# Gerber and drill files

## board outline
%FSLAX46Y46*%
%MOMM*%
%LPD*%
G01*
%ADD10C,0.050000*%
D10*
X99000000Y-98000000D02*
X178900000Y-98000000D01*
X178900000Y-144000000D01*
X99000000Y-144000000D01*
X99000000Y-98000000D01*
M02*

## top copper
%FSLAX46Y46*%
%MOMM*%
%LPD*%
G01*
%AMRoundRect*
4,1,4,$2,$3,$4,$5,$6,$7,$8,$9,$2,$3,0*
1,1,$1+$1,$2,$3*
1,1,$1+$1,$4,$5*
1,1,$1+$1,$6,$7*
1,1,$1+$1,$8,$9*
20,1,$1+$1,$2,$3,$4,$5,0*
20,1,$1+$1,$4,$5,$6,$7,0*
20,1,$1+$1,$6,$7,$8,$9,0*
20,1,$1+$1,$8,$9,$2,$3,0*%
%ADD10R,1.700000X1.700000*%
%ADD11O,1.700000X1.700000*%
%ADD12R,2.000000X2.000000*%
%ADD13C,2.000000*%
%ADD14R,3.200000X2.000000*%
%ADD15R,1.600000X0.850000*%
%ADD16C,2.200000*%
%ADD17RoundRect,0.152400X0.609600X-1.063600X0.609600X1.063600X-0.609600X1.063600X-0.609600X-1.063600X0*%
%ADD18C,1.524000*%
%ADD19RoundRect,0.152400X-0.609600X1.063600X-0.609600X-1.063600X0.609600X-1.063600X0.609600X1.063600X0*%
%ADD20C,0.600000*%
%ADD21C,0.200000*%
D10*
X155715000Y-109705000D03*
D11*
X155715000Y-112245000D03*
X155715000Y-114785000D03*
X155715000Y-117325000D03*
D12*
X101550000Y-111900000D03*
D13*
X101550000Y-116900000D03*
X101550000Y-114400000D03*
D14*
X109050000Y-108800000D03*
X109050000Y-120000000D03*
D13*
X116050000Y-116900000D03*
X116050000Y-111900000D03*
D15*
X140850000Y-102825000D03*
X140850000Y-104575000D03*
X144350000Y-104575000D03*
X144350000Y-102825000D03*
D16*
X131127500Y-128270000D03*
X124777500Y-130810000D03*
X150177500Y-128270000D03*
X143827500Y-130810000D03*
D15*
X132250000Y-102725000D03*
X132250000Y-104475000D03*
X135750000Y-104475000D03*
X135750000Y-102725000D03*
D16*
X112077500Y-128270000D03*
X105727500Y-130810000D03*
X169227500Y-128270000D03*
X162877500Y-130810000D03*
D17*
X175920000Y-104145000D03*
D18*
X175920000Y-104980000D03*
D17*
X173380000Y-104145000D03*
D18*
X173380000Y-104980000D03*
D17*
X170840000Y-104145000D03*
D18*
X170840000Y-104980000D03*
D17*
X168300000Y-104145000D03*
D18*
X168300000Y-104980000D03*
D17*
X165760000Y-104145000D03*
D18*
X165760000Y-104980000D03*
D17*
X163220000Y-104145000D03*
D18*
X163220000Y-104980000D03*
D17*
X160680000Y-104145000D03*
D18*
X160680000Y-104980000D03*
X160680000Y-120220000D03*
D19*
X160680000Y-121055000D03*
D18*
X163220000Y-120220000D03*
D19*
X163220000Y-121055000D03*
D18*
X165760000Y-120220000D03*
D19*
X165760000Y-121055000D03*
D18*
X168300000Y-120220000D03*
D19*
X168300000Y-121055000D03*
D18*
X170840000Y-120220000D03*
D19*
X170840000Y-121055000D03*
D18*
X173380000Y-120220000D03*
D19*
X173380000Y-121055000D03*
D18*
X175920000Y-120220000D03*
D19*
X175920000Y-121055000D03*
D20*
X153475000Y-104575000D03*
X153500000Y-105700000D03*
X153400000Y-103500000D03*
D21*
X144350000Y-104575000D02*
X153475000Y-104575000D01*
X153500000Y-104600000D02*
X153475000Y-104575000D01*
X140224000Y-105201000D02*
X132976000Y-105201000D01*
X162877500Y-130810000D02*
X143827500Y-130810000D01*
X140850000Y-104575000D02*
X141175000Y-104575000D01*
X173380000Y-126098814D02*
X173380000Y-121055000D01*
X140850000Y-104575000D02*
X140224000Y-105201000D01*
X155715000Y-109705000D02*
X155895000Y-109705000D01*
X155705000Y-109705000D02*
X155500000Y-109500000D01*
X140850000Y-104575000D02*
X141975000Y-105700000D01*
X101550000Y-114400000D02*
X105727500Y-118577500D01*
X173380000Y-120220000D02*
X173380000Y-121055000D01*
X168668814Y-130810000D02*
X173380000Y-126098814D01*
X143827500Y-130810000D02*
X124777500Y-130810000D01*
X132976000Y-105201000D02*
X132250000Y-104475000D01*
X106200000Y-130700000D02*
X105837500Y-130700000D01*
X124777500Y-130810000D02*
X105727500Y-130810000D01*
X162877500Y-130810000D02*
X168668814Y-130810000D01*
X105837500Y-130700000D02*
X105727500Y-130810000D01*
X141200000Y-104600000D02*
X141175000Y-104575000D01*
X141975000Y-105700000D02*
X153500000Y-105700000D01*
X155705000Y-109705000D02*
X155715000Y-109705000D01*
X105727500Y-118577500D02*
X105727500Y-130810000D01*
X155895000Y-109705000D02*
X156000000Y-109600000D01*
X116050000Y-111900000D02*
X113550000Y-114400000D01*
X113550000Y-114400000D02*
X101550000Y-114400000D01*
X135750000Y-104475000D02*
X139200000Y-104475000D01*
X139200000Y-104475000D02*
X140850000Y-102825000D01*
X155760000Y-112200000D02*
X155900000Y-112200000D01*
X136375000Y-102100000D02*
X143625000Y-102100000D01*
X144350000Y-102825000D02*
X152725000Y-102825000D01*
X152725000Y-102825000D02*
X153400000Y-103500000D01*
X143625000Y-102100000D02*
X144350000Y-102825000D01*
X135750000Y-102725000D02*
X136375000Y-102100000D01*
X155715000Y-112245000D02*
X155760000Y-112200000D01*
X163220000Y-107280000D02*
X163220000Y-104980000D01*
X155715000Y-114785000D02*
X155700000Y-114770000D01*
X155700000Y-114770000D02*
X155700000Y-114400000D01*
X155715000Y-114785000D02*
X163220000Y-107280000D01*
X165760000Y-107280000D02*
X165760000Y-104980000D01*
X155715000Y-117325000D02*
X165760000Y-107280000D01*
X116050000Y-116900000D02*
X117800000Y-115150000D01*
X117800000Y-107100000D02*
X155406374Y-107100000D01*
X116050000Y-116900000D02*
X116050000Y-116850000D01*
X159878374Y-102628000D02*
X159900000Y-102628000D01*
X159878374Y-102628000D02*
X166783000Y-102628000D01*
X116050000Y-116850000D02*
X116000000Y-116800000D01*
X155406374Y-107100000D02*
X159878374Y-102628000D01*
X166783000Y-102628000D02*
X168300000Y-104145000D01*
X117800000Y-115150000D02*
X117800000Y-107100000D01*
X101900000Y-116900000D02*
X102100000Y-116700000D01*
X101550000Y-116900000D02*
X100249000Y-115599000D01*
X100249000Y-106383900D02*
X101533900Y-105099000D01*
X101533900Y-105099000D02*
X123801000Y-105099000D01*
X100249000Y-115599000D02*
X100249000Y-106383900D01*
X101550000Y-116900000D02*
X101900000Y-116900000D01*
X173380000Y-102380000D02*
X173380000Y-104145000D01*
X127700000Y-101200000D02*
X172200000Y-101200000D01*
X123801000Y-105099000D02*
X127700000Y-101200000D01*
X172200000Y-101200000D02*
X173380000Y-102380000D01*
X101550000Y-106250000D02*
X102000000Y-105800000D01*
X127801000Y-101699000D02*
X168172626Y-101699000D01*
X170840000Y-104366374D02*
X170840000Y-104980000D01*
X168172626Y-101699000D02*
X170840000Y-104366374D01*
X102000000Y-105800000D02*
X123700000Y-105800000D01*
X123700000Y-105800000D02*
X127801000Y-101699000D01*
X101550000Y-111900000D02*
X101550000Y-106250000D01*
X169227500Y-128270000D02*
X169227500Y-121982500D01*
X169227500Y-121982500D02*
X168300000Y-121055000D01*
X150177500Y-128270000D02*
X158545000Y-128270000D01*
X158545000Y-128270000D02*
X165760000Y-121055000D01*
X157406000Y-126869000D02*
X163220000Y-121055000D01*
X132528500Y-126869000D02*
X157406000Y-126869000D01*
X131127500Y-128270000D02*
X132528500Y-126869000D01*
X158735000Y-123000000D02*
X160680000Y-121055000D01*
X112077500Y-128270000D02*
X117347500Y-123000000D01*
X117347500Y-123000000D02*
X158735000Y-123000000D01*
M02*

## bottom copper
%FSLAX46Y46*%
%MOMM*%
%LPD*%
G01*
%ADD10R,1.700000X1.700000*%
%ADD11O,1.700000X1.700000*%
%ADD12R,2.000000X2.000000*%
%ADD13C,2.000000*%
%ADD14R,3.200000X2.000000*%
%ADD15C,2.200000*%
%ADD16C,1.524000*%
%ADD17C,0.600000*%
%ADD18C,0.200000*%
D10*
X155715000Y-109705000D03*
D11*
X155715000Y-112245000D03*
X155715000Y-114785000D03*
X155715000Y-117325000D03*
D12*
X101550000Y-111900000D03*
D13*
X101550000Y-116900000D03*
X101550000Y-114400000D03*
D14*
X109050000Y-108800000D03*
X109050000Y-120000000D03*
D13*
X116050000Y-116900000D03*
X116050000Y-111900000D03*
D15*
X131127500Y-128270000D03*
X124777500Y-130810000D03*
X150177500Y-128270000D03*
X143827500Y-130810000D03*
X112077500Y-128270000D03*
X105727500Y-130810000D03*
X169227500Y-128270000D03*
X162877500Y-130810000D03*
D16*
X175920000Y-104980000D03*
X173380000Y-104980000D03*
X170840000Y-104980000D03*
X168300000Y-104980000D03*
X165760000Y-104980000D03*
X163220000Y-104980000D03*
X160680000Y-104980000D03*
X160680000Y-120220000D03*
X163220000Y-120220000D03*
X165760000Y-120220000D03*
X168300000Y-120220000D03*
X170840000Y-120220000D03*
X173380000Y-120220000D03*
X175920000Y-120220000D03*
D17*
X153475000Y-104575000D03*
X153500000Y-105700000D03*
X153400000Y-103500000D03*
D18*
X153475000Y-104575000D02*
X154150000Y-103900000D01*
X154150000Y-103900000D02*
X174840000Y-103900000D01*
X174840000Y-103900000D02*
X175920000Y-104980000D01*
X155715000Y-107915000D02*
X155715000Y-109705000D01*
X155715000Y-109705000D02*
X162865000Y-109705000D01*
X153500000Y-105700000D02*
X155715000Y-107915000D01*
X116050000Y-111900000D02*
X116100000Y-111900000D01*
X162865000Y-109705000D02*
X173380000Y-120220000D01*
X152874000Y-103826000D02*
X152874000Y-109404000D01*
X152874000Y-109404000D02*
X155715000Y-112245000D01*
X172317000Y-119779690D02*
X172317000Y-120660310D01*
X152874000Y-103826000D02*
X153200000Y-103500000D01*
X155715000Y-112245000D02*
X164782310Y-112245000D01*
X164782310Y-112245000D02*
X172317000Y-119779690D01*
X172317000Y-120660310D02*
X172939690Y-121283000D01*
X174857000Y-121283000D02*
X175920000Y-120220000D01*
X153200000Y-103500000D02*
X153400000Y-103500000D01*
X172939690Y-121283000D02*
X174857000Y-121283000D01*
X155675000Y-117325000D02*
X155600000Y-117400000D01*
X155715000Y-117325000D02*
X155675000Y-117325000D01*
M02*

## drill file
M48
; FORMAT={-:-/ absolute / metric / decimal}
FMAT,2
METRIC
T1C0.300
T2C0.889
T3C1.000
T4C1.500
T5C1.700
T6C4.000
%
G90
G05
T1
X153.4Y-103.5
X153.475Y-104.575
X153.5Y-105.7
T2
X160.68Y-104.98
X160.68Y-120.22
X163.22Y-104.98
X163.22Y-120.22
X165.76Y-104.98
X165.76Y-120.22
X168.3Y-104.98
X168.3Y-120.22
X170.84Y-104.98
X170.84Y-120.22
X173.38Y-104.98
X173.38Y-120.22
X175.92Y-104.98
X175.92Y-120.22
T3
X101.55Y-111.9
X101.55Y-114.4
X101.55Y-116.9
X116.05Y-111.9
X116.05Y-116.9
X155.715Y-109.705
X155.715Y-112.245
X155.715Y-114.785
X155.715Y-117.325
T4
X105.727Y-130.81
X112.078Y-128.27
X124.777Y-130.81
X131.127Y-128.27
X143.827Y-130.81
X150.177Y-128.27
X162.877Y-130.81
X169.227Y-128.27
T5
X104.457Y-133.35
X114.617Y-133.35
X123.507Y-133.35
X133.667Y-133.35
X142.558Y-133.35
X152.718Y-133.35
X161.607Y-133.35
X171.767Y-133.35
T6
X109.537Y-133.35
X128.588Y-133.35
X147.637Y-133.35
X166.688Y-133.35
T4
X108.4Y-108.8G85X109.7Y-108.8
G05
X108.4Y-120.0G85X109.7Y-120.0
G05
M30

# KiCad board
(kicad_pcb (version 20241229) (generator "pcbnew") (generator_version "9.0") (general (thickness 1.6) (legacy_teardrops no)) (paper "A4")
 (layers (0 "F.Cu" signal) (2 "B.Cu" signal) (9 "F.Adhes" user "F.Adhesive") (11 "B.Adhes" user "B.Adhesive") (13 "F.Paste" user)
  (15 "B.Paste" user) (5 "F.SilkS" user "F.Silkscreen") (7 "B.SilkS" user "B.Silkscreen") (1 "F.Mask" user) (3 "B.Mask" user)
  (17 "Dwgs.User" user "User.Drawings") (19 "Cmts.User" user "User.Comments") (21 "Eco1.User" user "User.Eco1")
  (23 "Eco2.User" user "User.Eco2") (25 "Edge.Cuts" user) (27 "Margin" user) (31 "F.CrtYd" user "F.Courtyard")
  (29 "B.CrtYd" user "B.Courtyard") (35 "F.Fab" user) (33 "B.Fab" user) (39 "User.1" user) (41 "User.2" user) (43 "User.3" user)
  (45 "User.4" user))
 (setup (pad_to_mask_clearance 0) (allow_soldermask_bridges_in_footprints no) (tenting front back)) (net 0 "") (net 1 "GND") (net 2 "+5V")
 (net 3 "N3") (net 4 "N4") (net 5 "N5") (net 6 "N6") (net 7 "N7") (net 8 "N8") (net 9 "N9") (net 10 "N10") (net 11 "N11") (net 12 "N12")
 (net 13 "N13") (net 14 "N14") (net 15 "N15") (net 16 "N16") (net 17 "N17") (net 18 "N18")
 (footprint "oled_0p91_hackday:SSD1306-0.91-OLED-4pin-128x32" (layer "F.Cu") (at 119.215 107.515)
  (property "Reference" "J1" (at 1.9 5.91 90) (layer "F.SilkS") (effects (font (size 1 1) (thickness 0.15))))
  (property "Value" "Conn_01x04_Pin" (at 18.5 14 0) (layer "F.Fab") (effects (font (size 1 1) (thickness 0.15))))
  (pad "1" thru_hole rect (at 36.5 2.19) (size 1.7 1.7) (drill 1) (layers "*.Cu" "*.Mask") (remove_unused_layers no) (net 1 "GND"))
  (pad "2" thru_hole oval (at 36.5 4.73) (size 1.7 1.7) (drill 1) (layers "*.Cu" "*.Mask") (remove_unused_layers no) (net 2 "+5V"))
  (pad "3" thru_hole oval (at 36.5 7.27) (size 1.7 1.7) (drill 1) (layers "*.Cu" "*.Mask") (remove_unused_layers no) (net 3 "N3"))
  (pad "4" thru_hole oval (at 36.5 9.81) (size 1.7 1.7) (drill 1) (layers "*.Cu" "*.Mask") (remove_unused_layers no) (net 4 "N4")))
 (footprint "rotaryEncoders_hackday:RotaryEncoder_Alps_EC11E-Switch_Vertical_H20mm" (layer "F.Cu") (at 101.55 111.9)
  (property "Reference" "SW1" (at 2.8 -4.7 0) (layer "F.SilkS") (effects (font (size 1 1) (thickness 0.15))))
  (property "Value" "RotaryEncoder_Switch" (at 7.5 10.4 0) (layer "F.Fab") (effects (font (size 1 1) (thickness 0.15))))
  (pad "A" thru_hole rect (at 0 0) (size 2 2) (drill 1) (layers "*.Cu" "*.Mask") (remove_unused_layers no) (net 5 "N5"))
  (pad "B" thru_hole circle (at 0 5) (size 2 2) (drill 1) (layers "*.Cu" "*.Mask") (remove_unused_layers no) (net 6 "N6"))
  (pad "C" thru_hole circle (at 0 2.5) (size 2 2) (drill 1) (layers "*.Cu" "*.Mask") (remove_unused_layers no) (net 1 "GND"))
  (pad "MP" thru_hole rect (at 7.5 -3.1) (size 3.2 2) (drill oval 2.8 1.5) (layers "*.Cu" "*.Mask") (remove_unused_layers no))
  (pad "MP" thru_hole rect (at 7.5 8.1) (size 3.2 2) (drill oval 2.8 1.5) (layers "*.Cu" "*.Mask") (remove_unused_layers no))
  (pad "S1" thru_hole circle (at 14.5 5) (size 2 2) (drill 1) (layers "*.Cu" "*.Mask") (remove_unused_layers no) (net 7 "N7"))
  (pad "S2" thru_hole circle (at 14.5 0) (size 2 2) (drill 1) (layers "*.Cu" "*.Mask") (remove_unused_layers no) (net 1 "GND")))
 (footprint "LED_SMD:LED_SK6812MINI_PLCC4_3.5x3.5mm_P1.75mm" (layer "F.Cu") (at 142.6 103.7)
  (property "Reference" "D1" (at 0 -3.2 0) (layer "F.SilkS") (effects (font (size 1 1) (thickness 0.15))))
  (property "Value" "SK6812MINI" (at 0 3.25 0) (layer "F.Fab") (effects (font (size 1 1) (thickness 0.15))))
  (pad "1" smd rect (at -1.75 -0.875) (size 1.6 0.85) (layers "F.Cu" "F.Mask" "F.Paste") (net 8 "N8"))
  (pad "2" smd rect (at -1.75 0.875) (size 1.6 0.85) (layers "F.Cu" "F.Mask" "F.Paste") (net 1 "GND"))
  (pad "3" smd rect (at 1.75 0.875) (size 1.6 0.85) (layers "F.Cu" "F.Mask" "F.Paste") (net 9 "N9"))
  (pad "4" smd rect (at 1.75 -0.875) (size 1.6 0.85) (layers "F.Cu" "F.Mask" "F.Paste") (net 2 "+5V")))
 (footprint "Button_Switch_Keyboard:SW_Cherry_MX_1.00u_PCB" (layer "F.Cu") (at 131.1275 128.27)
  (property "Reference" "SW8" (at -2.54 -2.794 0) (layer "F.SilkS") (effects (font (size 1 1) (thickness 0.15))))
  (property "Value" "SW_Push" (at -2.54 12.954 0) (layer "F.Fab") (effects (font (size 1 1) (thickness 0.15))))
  (pad "" np_thru_hole circle (at -7.62 5.08) (size 1.7 1.7) (drill 1.7) (layers "*.Cu" "*.Mask"))
  (pad "" np_thru_hole circle (at -2.54 5.08) (size 4 4) (drill 4) (layers "*.Cu" "*.Mask"))
  (pad "" np_thru_hole circle (at 2.54 5.08) (size 1.7 1.7) (drill 1.7) (layers "*.Cu" "*.Mask"))
  (pad "1" thru_hole circle (at 0 0) (size 2.2 2.2) (drill 1.5) (layers "*.Cu" "*.Mask") (remove_unused_layers no) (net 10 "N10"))
  (pad "2" thru_hole circle (at -6.35 2.54) (size 2.2 2.2) (drill 1.5) (layers "*.Cu" "*.Mask") (remove_unused_layers no) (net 1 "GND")))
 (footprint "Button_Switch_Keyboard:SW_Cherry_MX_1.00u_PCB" (layer "F.Cu") (at 150.1775 128.27)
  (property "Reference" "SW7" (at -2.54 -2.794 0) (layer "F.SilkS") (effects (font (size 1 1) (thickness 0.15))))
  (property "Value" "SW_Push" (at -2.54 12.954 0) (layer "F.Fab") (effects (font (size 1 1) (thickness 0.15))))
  (pad "" np_thru_hole circle (at -7.62 5.08) (size 1.7 1.7) (drill 1.7) (layers "*.Cu" "*.Mask"))
  (pad "" np_thru_hole circle (at -2.54 5.08) (size 4 4) (drill 4) (layers "*.Cu" "*.Mask"))
  (pad "" np_thru_hole circle (at 2.54 5.08) (size 1.7 1.7) (drill 1.7) (layers "*.Cu" "*.Mask"))
  (pad "1" thru_hole circle (at 0 0) (size 2.2 2.2) (drill 1.5) (layers "*.Cu" "*.Mask") (remove_unused_layers no) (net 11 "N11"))
  (pad "2" thru_hole circle (at -6.35 2.54) (size 2.2 2.2) (drill 1.5) (layers "*.Cu" "*.Mask") (remove_unused_layers no) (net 1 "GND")))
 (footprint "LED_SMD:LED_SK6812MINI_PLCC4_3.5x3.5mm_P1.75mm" (layer "F.Cu") (at 134 103.6)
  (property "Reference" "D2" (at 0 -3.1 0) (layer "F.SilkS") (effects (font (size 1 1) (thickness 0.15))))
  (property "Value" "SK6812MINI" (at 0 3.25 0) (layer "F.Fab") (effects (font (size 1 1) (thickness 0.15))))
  (pad "1" smd rect (at -1.75 -0.875) (size 1.6 0.85) (layers "F.Cu" "F.Mask" "F.Paste") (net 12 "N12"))
  (pad "2" smd rect (at -1.75 0.875) (size 1.6 0.85) (layers "F.Cu" "F.Mask" "F.Paste") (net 1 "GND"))
  (pad "3" smd rect (at 1.75 0.875) (size 1.6 0.85) (layers "F.Cu" "F.Mask" "F.Paste") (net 8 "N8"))
  (pad "4" smd rect (at 1.75 -0.875) (size 1.6 0.85) (layers "F.Cu" "F.Mask" "F.Paste") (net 2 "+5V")))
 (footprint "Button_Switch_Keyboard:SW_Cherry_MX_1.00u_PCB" (layer "F.Cu") (at 112.0775 128.27)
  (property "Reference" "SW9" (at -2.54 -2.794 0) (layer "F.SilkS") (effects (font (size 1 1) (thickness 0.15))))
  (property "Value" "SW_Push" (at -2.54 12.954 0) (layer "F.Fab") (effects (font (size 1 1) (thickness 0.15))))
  (pad "" np_thru_hole circle (at -7.62 5.08) (size 1.7 1.7) (drill 1.7) (layers "*.Cu" "*.Mask"))
  (pad "" np_thru_hole circle (at -2.54 5.08) (size 4 4) (drill 4) (layers "*.Cu" "*.Mask"))
  (pad "" np_thru_hole circle (at 2.54 5.08) (size 1.7 1.7) (drill 1.7) (layers "*.Cu" "*.Mask"))
  (pad "1" thru_hole circle (at 0 0) (size 2.2 2.2) (drill 1.5) (layers "*.Cu" "*.Mask") (remove_unused_layers no) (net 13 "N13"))
  (pad "2" thru_hole circle (at -6.35 2.54) (size 2.2 2.2) (drill 1.5) (layers "*.Cu" "*.Mask") (remove_unused_layers no) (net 1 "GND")))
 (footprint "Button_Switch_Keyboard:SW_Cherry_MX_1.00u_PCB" (layer "F.Cu") (at 169.2275 128.27)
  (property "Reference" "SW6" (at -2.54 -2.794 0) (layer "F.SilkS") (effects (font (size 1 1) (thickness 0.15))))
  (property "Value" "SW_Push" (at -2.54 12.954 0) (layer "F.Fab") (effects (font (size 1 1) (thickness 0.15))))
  (pad "" np_thru_hole circle (at -7.62 5.08) (size 1.7 1.7) (drill 1.7) (layers "*.Cu" "*.Mask"))
  (pad "" np_thru_hole circle (at -2.54 5.08) (size 4 4) (drill 4) (layers "*.Cu" "*.Mask"))
  (pad "" np_thru_hole circle (at 2.54 5.08) (size 1.7 1.7) (drill 1.7) (layers "*.Cu" "*.Mask"))
  (pad "1" thru_hole circle (at 0 0) (size 2.2 2.2) (drill 1.5) (layers "*.Cu" "*.Mask") (remove_unused_layers no) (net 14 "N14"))
  (pad "2" thru_hole circle (at -6.35 2.54) (size 2.2 2.2) (drill 1.5) (layers "*.Cu" "*.Mask") (remove_unused_layers no) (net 1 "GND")))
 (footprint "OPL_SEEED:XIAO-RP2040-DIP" (layer "F.Cu") (at 168.3 112.6 -90)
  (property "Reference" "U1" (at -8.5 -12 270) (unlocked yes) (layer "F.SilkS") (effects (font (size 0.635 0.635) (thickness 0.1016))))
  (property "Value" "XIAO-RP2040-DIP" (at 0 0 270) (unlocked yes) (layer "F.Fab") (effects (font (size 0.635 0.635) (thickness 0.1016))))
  (pad "1" smd roundrect (at -8.455 -7.62 90) (size 2.432 1.524) (layers "F.Cu" "F.Mask") (roundrect_rratio 0.1) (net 9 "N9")
   (thermal_bridge_angle 45))
  (pad "1" thru_hole circle (at -7.62 -7.62 90) (size 1.524 1.524) (drill 0.889) (layers "*.Cu" "*.Mask") (remove_unused_layers no)
   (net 9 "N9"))
  (pad "2" smd roundrect (at -8.455 -5.08 90) (size 2.432 1.524) (layers "F.Cu" "F.Mask") (roundrect_rratio 0.1) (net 6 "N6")
   (thermal_bridge_angle 45))
  (pad "2" thru_hole circle (at -7.62 -5.08 90) (size 1.524 1.524) (drill 0.889) (layers "*.Cu" "*.Mask") (remove_unused_layers no)
   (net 6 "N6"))
  (pad "3" smd roundrect (at -8.455 -2.54 90) (size 2.432 1.524) (layers "F.Cu" "F.Mask") (roundrect_rratio 0.1) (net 5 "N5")
   (thermal_bridge_angle 45))
  (pad "3" thru_hole circle (at -7.62 -2.54 90) (size 1.524 1.524) (drill 0.889) (layers "*.Cu" "*.Mask") (remove_unused_layers no)
   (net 5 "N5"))
  (pad "4" smd roundrect (at -8.455 0 90) (size 2.432 1.524) (layers "F.Cu" "F.Mask") (roundrect_rratio 0.1) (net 7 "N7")
   (thermal_bridge_angle 45))
  (pad "4" thru_hole circle (at -7.62 0 90) (size 1.524 1.524) (drill 0.889) (layers "*.Cu" "*.Mask") (remove_unused_layers no) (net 7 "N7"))
  (pad "5" smd roundrect (at -8.455 2.54 90) (size 2.432 1.524) (layers "F.Cu" "F.Mask") (roundrect_rratio 0.1) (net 4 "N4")
   (thermal_bridge_angle 45))
  (pad "5" thru_hole circle (at -7.62 2.54 90) (size 1.524 1.524) (drill 0.889) (layers "*.Cu" "*.Mask") (remove_unused_layers no)
   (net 4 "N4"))
  (pad "6" smd roundrect (at -8.455 5.08 90) (size 2.432 1.524) (layers "F.Cu" "F.Mask") (roundrect_rratio 0.1) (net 3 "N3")
   (thermal_bridge_angle 45))
  (pad "6" thru_hole circle (at -7.62 5.08 90) (size 1.524 1.524) (drill 0.889) (layers "*.Cu" "*.Mask") (remove_unused_layers no)
   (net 3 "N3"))
  (pad "7" smd roundrect (at -8.455 7.62 90) (size 2.432 1.524) (layers "F.Cu" "F.Mask") (roundrect_rratio 0.1) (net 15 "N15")
   (thermal_bridge_angle 45))
  (pad "7" thru_hole circle (at -7.62 7.62 90) (size 1.524 1.524) (drill 0.889) (layers "*.Cu" "*.Mask") (remove_unused_layers no)
   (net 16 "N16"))
  (pad "8" thru_hole circle (at 7.62 7.62 270) (size 1.524 1.524) (drill 0.889) (layers "*.Cu" "*.Mask") (remove_unused_layers no)
   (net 13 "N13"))
  (pad "8" smd roundrect (at 8.455 7.62 270) (size 2.432 1.524) (layers "F.Cu" "F.Mask") (roundrect_rratio 0.1) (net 13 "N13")
   (thermal_bridge_angle 45))
  (pad "9" thru_hole circle (at 7.62 5.08 270) (size 1.524 1.524) (drill 0.889) (layers "*.Cu" "*.Mask") (remove_unused_layers no)
   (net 10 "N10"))
  (pad "9" smd roundrect (at 8.455 5.08 270) (size 2.432 1.524) (layers "F.Cu" "F.Mask") (roundrect_rratio 0.1) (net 10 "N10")
   (thermal_bridge_angle 45))
  (pad "10" thru_hole circle (at 7.62 2.54 270) (size 1.524 1.524) (drill 0.889) (layers "*.Cu" "*.Mask") (remove_unused_layers no)
   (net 11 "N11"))
  (pad "10" smd roundrect (at 8.455 2.54 270) (size 2.432 1.524) (layers "F.Cu" "F.Mask") (roundrect_rratio 0.1) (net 11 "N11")
   (thermal_bridge_angle 45))
  (pad "11" thru_hole circle (at 7.62 0 270) (size 1.524 1.524) (drill 0.889) (layers "*.Cu" "*.Mask") (remove_unused_layers no)
   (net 14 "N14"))
  (pad "11" smd roundrect (at 8.455 0 270) (size 2.432 1.524) (layers "F.Cu" "F.Mask") (roundrect_rratio 0.1) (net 14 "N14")
   (thermal_bridge_angle 45))
  (pad "12" thru_hole circle (at 7.62 -2.54 270) (size 1.524 1.524) (drill 0.889) (layers "*.Cu" "*.Mask") (remove_unused_layers no)
   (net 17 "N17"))
  (pad "12" smd roundrect (at 8.455 -2.54 270) (size 2.432 1.524) (layers "F.Cu" "F.Mask") (roundrect_rratio 0.1) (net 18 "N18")
   (thermal_bridge_angle 45))
  (pad "13" thru_hole circle (at 7.62 -5.08 270) (size 1.524 1.524) (drill 0.889) (layers "*.Cu" "*.Mask") (remove_unused_layers no)
   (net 1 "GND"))
  (pad "13" smd roundrect (at 8.455 -5.08 270) (size 2.432 1.524) (layers "F.Cu" "F.Mask") (roundrect_rratio 0.1) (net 1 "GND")
   (thermal_bridge_angle 45))
  (pad "14" thru_hole circle (at 7.62 -7.62 270) (size 1.524 1.524) (drill 0.889) (layers "*.Cu" "*.Mask") (remove_unused_layers no)
   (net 2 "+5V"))
  (pad "14" smd roundrect (at 8.455 -7.62 270) (size 2.432 1.524) (layers "F.Cu" "F.Mask") (roundrect_rratio 0.1) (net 2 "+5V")
   (thermal_bridge_angle 45)))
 (gr_rect (start 99 98) (end 178.9 144) (stroke (width 0.05) (type default)) (fill no) (layer "Edge.Cuts"))
 (segment (start 144.35 104.575) (end 153.475 104.575) (width 0.2) (layer "F.Cu") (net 9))
 (segment (start 153.5 104.6) (end 153.475 104.575) (width 0.2) (layer "F.Cu") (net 9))
 (via (at 153.475 104.575) (size 0.6) (drill 0.3) (layers "F.Cu" "B.Cu") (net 9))
 (segment (start 153.475 104.575) (end 154.15 103.9) (width 0.2) (layer "B.Cu") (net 9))
 (segment (start 154.15 103.9) (end 174.84 103.9) (width 0.2) (layer "B.Cu") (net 9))
 (segment (start 174.84 103.9) (end 175.92 104.98) (width 0.2) (layer "B.Cu") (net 9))
 (segment (start 140.224 105.201) (end 132.976 105.201) (width 0.2) (layer "F.Cu") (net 1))
 (segment (start 162.8775 130.81) (end 143.8275 130.81) (width 0.2) (layer "F.Cu") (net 1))
 (segment (start 140.85 104.575) (end 141.175 104.575) (width 0.2) (layer "F.Cu") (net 1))
 (segment (start 173.38 126.098814) (end 173.38 121.055) (width 0.2) (layer "F.Cu") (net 1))
 (segment (start 140.85 104.575) (end 140.224 105.201) (width 0.2) (layer "F.Cu") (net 1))
 (segment (start 155.715 109.705) (end 155.895 109.705) (width 0.2) (layer "F.Cu") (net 1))
 (segment (start 155.705 109.705) (end 155.5 109.5) (width 0.2) (layer "F.Cu") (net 1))
 (segment (start 140.85 104.575) (end 141.975 105.7) (width 0.2) (layer "F.Cu") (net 1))
 (segment (start 101.55 114.4) (end 105.7275 118.5775) (width 0.2) (layer "F.Cu") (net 1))
 (segment (start 173.38 120.22) (end 173.38 121.055) (width 0.2) (layer "F.Cu") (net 1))
 (segment (start 168.668814 130.81) (end 173.38 126.098814) (width 0.2) (layer "F.Cu") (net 1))
 (segment (start 143.8275 130.81) (end 124.7775 130.81) (width 0.2) (layer "F.Cu") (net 1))
 (segment (start 132.976 105.201) (end 132.25 104.475) (width 0.2) (layer "F.Cu") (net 1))
 (segment (start 106.2 130.7) (end 105.8375 130.7) (width 0.2) (layer "F.Cu") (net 1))
 (segment (start 124.7775 130.81) (end 105.7275 130.81) (width 0.2) (layer "F.Cu") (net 1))
 (segment (start 162.8775 130.81) (end 168.668814 130.81) (width 0.2) (layer "F.Cu") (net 1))
 (segment (start 105.8375 130.7) (end 105.7275 130.81) (width 0.2) (layer "F.Cu") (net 1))
 (segment (start 141.2 104.6) (end 141.175 104.575) (width 0.2) (layer "F.Cu") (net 1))
 (segment (start 141.975 105.7) (end 153.5 105.7) (width 0.2) (layer "F.Cu") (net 1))
 (segment (start 155.705 109.705) (end 155.715 109.705) (width 0.2) (layer "F.Cu") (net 1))
 (segment (start 105.7275 118.5775) (end 105.7275 130.81) (width 0.2) (layer "F.Cu") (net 1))
 (segment (start 155.895 109.705) (end 156 109.6) (width 0.2) (layer "F.Cu") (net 1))
 (segment (start 116.05 111.9) (end 113.55 114.4) (width 0.2) (layer "F.Cu") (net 1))
 (segment (start 113.55 114.4) (end 101.55 114.4) (width 0.2) (layer "F.Cu") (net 1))
 (via (at 153.5 105.7) (size 0.6) (drill 0.3) (layers "F.Cu" "B.Cu") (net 1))
 (segment (start 155.715 107.915) (end 155.715 109.705) (width 0.2) (layer "B.Cu") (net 1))
 (segment (start 155.715 109.705) (end 162.865 109.705) (width 0.2) (layer "B.Cu") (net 1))
 (segment (start 153.5 105.7) (end 155.715 107.915) (width 0.2) (layer "B.Cu") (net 1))
 (segment (start 116.05 111.9) (end 116.1 111.9) (width 0.2) (layer "B.Cu") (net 1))
 (segment (start 162.865 109.705) (end 173.38 120.22) (width 0.2) (layer "B.Cu") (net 1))
 (segment (start 135.75 104.475) (end 139.2 104.475) (width 0.2) (layer "F.Cu") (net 8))
 (segment (start 139.2 104.475) (end 140.85 102.825) (width 0.2) (layer "F.Cu") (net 8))
 (segment (start 155.76 112.2) (end 155.9 112.2) (width 0.2) (layer "F.Cu") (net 2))
 (segment (start 136.375 102.1) (end 143.625 102.1) (width 0.2) (layer "F.Cu") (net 2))
 (segment (start 144.35 102.825) (end 152.725 102.825) (width 0.2) (layer "F.Cu") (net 2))
 (segment (start 152.725 102.825) (end 153.4 103.5) (width 0.2) (layer "F.Cu") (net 2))
 (segment (start 143.625 102.1) (end 144.35 102.825) (width 0.2) (layer "F.Cu") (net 2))
 (segment (start 135.75 102.725) (end 136.375 102.1) (width 0.2) (layer "F.Cu") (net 2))
 (segment (start 155.715 112.245) (end 155.76 112.2) (width 0.2) (layer "F.Cu") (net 2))
 (via (at 153.4 103.5) (size 0.6) (drill 0.3) (layers "F.Cu" "B.Cu") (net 2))
 (segment (start 152.874 103.826) (end 152.874 109.404) (width 0.2) (layer "B.Cu") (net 2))
 (segment (start 152.874 109.404) (end 155.715 112.245) (width 0.2) (layer "B.Cu") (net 2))
 (segment (start 172.317 119.77969) (end 172.317 120.66031) (width 0.2) (layer "B.Cu") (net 2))
 (segment (start 152.874 103.826) (end 153.2 103.5) (width 0.2) (layer "B.Cu") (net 2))
 (segment (start 155.715 112.245) (end 164.78231 112.245) (width 0.2) (layer "B.Cu") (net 2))
 (segment (start 164.78231 112.245) (end 172.317 119.77969) (width 0.2) (layer "B.Cu") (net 2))
 (segment (start 172.317 120.66031) (end 172.93969 121.283) (width 0.2) (layer "B.Cu") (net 2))
 (segment (start 174.857 121.283) (end 175.92 120.22) (width 0.2) (layer "B.Cu") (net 2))
 (segment (start 153.2 103.5) (end 153.4 103.5) (width 0.2) (layer "B.Cu") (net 2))
 (segment (start 172.93969 121.283) (end 174.857 121.283) (width 0.2) (layer "B.Cu") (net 2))
 (segment (start 163.22 107.28) (end 163.22 104.98) (width 0.2) (layer "F.Cu") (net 3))
 (segment (start 155.715 114.785) (end 155.7 114.77) (width 0.2) (layer "F.Cu") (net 3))
 (segment (start 155.7 114.77) (end 155.7 114.4) (width 0.2) (layer "F.Cu") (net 3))
 (segment (start 155.715 114.785) (end 163.22 107.28) (width 0.2) (layer "F.Cu") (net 3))
 (segment (start 165.76 107.28) (end 165.76 104.98) (width 0.2) (layer "F.Cu") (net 4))
 (segment (start 155.715 117.325) (end 165.76 107.28) (width 0.2) (layer "F.Cu") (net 4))
 (segment (start 155.675 117.325) (end 155.6 117.4) (width 0.2) (layer "B.Cu") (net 4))
 (segment (start 155.715 117.325) (end 155.675 117.325) (width 0.2) (layer "B.Cu") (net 4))
 (segment (start 116.05 116.9) (end 117.8 115.15) (width 0.2) (layer "F.Cu") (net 7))
 (segment (start 117.8 107.1) (end 155.406374 107.1) (width 0.2) (layer "F.Cu") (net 7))
 (segment (start 116.05 116.9) (end 116.05 116.85) (width 0.2) (layer "F.Cu") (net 7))
 (segment (start 159.878374 102.628) (end 159.9 102.628) (width 0.2) (layer "F.Cu") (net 7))
 (segment (start 159.878374 102.628) (end 166.783 102.628) (width 0.2) (layer "F.Cu") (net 7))
 (segment (start 116.05 116.85) (end 116 116.8) (width 0.2) (layer "F.Cu") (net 7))
 (segment (start 155.406374 107.1) (end 159.878374 102.628) (width 0.2) (layer "F.Cu") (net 7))
 (segment (start 166.783 102.628) (end 168.3 104.145) (width 0.2) (layer "F.Cu") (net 7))
 (segment (start 117.8 115.15) (end 117.8 107.1) (width 0.2) (layer "F.Cu") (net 7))
 (segment (start 101.9 116.9) (end 102.1 116.7) (width 0.2) (layer "F.Cu") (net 6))
 (segment (start 101.55 116.9) (end 100.249 115.599) (width 0.2) (layer "F.Cu") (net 6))
 (segment (start 100.249 106.3839) (end 101.5339 105.099) (width 0.2) (layer "F.Cu") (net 6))
 (segment (start 101.5339 105.099) (end 123.801 105.099) (width 0.2) (layer "F.Cu") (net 6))
 (segment (start 100.249 115.599) (end 100.249 106.3839) (width 0.2) (layer "F.Cu") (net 6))
 (segment (start 101.55 116.9) (end 101.9 116.9) (width 0.2) (layer "F.Cu") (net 6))
 (segment (start 173.38 102.38) (end 173.38 104.145) (width 0.2) (layer "F.Cu") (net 6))
 (segment (start 127.7 101.2) (end 172.2 101.2) (width 0.2) (layer "F.Cu") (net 6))
 (segment (start 123.801 105.099) (end 127.7 101.2) (width 0.2) (layer "F.Cu") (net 6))
 (segment (start 172.2 101.2) (end 173.38 102.38) (width 0.2) (layer "F.Cu") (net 6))
 (segment (start 101.55 106.25) (end 102 105.8) (width 0.2) (layer "F.Cu") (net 5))
 (segment (start 127.801 101.699) (end 168.172626 101.699) (width 0.2) (layer "F.Cu") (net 5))
 (segment (start 170.84 104.366374) (end 170.84 104.98) (width 0.2) (layer "F.Cu") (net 5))
 (segment (start 168.172626 101.699) (end 170.84 104.366374) (width 0.2) (layer "F.Cu") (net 5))
 (segment (start 102 105.8) (end 123.7 105.8) (width 0.2) (layer "F.Cu") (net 5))
 (segment (start 123.7 105.8) (end 127.801 101.699) (width 0.2) (layer "F.Cu") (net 5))
 (segment (start 101.55 111.9) (end 101.55 106.25) (width 0.2) (layer "F.Cu") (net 5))
 (segment (start 169.2275 128.27) (end 169.2275 121.9825) (width 0.2) (layer "F.Cu") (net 14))
 (segment (start 169.2275 121.9825) (end 168.3 121.055) (width 0.2) (layer "F.Cu") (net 14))
 (segment (start 150.1775 128.27) (end 158.545 128.27) (width 0.2) (layer "F.Cu") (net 11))
 (segment (start 158.545 128.27) (end 165.76 121.055) (width 0.2) (layer "F.Cu") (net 11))
 (segment (start 157.406 126.869) (end 163.22 121.055) (width 0.2) (layer "F.Cu") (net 10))
 (segment (start 132.5285 126.869) (end 157.406 126.869) (width 0.2) (layer "F.Cu") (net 10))
 (segment (start 131.1275 128.27) (end 132.5285 126.869) (width 0.2) (layer "F.Cu") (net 10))
 (segment (start 158.735 123) (end 160.68 121.055) (width 0.2) (layer "F.Cu") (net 13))
 (segment (start 112.0775 128.27) (end 117.3475 123) (width 0.2) (layer "F.Cu") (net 13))
 (segment (start 117.3475 123) (end 158.735 123) (width 0.2) (layer "F.Cu") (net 13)))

